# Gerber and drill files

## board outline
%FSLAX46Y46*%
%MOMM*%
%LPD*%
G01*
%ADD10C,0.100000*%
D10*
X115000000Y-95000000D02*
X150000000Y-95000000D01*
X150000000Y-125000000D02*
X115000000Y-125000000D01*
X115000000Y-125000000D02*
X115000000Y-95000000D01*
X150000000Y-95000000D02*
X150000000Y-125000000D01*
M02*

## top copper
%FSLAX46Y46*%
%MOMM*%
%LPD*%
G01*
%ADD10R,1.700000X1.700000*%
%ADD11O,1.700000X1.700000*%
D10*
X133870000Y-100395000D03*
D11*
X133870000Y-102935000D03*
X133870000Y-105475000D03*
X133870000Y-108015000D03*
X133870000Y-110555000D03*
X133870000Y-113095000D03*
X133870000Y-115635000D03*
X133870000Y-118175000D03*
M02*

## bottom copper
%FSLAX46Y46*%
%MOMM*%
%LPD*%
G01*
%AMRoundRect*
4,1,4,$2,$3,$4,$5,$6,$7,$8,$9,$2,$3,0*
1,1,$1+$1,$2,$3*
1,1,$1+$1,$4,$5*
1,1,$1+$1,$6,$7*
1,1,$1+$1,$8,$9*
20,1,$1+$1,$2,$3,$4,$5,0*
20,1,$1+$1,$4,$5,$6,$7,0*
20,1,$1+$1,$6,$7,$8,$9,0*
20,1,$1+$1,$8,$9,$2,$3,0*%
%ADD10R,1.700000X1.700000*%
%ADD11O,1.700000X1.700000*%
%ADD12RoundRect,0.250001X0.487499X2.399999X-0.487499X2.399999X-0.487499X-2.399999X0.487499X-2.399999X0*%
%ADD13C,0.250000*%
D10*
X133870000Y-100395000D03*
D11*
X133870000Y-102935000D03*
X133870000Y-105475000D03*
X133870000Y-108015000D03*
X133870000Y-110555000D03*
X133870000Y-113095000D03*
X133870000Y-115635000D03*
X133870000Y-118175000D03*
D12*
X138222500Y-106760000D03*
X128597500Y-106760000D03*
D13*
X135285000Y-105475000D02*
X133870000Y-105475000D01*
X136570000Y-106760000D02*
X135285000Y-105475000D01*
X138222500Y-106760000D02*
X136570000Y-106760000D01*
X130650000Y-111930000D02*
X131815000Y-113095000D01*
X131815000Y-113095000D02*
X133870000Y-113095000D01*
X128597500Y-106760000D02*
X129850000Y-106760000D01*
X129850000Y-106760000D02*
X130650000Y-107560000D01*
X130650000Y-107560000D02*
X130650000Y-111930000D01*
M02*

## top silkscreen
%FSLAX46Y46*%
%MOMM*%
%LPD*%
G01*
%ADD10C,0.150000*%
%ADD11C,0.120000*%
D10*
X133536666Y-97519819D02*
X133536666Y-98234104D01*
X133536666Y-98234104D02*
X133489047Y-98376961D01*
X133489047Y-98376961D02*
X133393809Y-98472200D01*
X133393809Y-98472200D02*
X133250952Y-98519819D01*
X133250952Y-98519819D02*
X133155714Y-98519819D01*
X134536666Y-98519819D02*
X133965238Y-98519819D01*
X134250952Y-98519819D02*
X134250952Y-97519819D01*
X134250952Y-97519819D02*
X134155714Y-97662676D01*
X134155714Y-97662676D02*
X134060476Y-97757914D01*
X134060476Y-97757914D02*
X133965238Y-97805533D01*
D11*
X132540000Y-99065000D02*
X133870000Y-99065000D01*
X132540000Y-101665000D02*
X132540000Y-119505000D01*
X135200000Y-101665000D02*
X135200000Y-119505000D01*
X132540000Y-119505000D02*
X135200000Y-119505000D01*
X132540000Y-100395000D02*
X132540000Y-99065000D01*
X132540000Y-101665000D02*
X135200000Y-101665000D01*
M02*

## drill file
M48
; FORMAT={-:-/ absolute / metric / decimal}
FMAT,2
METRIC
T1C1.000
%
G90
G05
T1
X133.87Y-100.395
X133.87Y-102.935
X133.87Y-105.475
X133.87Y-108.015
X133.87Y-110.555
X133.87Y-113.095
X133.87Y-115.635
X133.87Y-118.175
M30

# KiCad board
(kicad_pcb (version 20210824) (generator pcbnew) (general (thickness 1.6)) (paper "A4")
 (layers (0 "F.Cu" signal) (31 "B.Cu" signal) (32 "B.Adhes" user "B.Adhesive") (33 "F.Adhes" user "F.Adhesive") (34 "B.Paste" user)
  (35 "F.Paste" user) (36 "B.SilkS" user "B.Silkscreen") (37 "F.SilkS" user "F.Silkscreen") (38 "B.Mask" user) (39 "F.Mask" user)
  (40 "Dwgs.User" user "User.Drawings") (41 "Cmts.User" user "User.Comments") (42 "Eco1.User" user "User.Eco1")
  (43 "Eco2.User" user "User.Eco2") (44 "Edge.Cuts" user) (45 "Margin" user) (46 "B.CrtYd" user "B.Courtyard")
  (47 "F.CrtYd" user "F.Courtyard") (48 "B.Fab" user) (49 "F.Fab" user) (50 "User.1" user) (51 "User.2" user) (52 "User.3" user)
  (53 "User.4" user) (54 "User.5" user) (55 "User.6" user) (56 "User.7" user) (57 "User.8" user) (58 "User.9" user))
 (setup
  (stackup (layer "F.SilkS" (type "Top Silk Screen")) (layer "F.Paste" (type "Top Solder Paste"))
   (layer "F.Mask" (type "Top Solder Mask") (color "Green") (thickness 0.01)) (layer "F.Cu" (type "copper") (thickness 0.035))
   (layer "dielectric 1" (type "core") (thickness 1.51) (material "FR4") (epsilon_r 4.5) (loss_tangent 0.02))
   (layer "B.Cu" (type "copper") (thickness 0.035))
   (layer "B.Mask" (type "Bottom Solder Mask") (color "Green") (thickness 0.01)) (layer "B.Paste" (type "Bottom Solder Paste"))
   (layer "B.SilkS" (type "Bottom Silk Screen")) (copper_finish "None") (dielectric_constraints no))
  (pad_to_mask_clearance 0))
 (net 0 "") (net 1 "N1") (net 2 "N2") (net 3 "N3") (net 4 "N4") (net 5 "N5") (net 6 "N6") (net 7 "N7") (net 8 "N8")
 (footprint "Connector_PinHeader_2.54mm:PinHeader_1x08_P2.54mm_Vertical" (layer "F.Cu") (at 133.87 100.395)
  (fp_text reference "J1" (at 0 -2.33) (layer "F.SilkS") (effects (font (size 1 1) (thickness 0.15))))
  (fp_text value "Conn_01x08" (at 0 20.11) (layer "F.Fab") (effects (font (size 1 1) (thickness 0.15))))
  (fp_line (start -1.33 -1.33) (end 0 -1.33) (layer "F.SilkS") (width 0.12))
  (fp_line (start -1.33 1.27) (end -1.33 19.11) (layer "F.SilkS") (width 0.12))
  (fp_line (start 1.33 1.27) (end 1.33 19.11) (layer "F.SilkS") (width 0.12))
  (fp_line (start -1.33 19.11) (end 1.33 19.11) (layer "F.SilkS") (width 0.12))
  (fp_line (start -1.33 0) (end -1.33 -1.33) (layer "F.SilkS") (width 0.12))
  (fp_line (start -1.33 1.27) (end 1.33 1.27) (layer "F.SilkS") (width 0.12))
  (pad "1" thru_hole rect locked (at 0 0) (size 1.7 1.7) (drill 1) (layers *.Cu *.Mask) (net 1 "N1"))
  (pad "2" thru_hole oval locked (at 0 2.54) (size 1.7 1.7) (drill 1) (layers *.Cu *.Mask) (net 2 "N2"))
  (pad "3" thru_hole oval locked (at 0 5.08) (size 1.7 1.7) (drill 1) (layers *.Cu *.Mask) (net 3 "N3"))
  (pad "4" thru_hole oval locked (at 0 7.62) (size 1.7 1.7) (drill 1) (layers *.Cu *.Mask) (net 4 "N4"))
  (pad "5" thru_hole oval locked (at 0 10.16) (size 1.7 1.7) (drill 1) (layers *.Cu *.Mask) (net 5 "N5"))
  (pad "6" thru_hole oval locked (at 0 12.7) (size 1.7 1.7) (drill 1) (layers *.Cu *.Mask) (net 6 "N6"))
  (pad "7" thru_hole oval locked (at 0 15.24) (size 1.7 1.7) (drill 1) (layers *.Cu *.Mask) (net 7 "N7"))
  (pad "8" thru_hole oval locked (at 0 17.78) (size 1.7 1.7) (drill 1) (layers *.Cu *.Mask) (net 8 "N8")))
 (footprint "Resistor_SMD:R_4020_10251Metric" (layer "B.Cu") (at 133.41 106.76 180)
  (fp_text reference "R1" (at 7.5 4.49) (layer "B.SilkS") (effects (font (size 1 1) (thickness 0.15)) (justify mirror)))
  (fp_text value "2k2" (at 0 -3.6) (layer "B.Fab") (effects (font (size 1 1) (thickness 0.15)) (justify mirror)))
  (pad "1" smd roundrect locked (at -4.8125 0 180) (size 1.475 5.3) (layers "B.Cu" "B.Paste" "B.Mask") (roundrect_rratio 0.169492)
   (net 3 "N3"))
  (pad "2" smd roundrect locked (at 4.8125 0 180) (size 1.475 5.3) (layers "B.Cu" "B.Paste" "B.Mask") (roundrect_rratio 0.169492)
   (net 6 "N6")))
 (gr_line (start 115 95) (end 150 95) (layer "Edge.Cuts") (width 0.1))
 (gr_line (start 150 125) (end 115 125) (layer "Edge.Cuts") (width 0.1))
 (gr_line (start 115 125) (end 115 95) (layer "Edge.Cuts") (width 0.1))
 (gr_line (start 150 95) (end 150 125) (layer "Edge.Cuts") (width 0.1))
 (segment (start 135.285 105.475) (end 133.87 105.475) (width 0.25) (layer "B.Cu") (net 3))
 (segment (start 136.57 106.76) (end 135.285 105.475) (width 0.25) (layer "B.Cu") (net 3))
 (segment (start 138.2225 106.76) (end 136.57 106.76) (width 0.25) (layer "B.Cu") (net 3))
 (segment (start 130.65 111.93) (end 131.815 113.095) (width 0.25) (layer "B.Cu") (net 6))
 (segment (start 131.815 113.095) (end 133.87 113.095) (width 0.25) (layer "B.Cu") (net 6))
 (segment (start 128.5975 106.76) (end 129.85 106.76) (width 0.25) (layer "B.Cu") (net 6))
 (segment (start 129.85 106.76) (end 130.65 107.56) (width 0.25) (layer "B.Cu") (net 6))
 (segment (start 130.65 107.56) (end 130.65 111.93) (width 0.25) (layer "B.Cu") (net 6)))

